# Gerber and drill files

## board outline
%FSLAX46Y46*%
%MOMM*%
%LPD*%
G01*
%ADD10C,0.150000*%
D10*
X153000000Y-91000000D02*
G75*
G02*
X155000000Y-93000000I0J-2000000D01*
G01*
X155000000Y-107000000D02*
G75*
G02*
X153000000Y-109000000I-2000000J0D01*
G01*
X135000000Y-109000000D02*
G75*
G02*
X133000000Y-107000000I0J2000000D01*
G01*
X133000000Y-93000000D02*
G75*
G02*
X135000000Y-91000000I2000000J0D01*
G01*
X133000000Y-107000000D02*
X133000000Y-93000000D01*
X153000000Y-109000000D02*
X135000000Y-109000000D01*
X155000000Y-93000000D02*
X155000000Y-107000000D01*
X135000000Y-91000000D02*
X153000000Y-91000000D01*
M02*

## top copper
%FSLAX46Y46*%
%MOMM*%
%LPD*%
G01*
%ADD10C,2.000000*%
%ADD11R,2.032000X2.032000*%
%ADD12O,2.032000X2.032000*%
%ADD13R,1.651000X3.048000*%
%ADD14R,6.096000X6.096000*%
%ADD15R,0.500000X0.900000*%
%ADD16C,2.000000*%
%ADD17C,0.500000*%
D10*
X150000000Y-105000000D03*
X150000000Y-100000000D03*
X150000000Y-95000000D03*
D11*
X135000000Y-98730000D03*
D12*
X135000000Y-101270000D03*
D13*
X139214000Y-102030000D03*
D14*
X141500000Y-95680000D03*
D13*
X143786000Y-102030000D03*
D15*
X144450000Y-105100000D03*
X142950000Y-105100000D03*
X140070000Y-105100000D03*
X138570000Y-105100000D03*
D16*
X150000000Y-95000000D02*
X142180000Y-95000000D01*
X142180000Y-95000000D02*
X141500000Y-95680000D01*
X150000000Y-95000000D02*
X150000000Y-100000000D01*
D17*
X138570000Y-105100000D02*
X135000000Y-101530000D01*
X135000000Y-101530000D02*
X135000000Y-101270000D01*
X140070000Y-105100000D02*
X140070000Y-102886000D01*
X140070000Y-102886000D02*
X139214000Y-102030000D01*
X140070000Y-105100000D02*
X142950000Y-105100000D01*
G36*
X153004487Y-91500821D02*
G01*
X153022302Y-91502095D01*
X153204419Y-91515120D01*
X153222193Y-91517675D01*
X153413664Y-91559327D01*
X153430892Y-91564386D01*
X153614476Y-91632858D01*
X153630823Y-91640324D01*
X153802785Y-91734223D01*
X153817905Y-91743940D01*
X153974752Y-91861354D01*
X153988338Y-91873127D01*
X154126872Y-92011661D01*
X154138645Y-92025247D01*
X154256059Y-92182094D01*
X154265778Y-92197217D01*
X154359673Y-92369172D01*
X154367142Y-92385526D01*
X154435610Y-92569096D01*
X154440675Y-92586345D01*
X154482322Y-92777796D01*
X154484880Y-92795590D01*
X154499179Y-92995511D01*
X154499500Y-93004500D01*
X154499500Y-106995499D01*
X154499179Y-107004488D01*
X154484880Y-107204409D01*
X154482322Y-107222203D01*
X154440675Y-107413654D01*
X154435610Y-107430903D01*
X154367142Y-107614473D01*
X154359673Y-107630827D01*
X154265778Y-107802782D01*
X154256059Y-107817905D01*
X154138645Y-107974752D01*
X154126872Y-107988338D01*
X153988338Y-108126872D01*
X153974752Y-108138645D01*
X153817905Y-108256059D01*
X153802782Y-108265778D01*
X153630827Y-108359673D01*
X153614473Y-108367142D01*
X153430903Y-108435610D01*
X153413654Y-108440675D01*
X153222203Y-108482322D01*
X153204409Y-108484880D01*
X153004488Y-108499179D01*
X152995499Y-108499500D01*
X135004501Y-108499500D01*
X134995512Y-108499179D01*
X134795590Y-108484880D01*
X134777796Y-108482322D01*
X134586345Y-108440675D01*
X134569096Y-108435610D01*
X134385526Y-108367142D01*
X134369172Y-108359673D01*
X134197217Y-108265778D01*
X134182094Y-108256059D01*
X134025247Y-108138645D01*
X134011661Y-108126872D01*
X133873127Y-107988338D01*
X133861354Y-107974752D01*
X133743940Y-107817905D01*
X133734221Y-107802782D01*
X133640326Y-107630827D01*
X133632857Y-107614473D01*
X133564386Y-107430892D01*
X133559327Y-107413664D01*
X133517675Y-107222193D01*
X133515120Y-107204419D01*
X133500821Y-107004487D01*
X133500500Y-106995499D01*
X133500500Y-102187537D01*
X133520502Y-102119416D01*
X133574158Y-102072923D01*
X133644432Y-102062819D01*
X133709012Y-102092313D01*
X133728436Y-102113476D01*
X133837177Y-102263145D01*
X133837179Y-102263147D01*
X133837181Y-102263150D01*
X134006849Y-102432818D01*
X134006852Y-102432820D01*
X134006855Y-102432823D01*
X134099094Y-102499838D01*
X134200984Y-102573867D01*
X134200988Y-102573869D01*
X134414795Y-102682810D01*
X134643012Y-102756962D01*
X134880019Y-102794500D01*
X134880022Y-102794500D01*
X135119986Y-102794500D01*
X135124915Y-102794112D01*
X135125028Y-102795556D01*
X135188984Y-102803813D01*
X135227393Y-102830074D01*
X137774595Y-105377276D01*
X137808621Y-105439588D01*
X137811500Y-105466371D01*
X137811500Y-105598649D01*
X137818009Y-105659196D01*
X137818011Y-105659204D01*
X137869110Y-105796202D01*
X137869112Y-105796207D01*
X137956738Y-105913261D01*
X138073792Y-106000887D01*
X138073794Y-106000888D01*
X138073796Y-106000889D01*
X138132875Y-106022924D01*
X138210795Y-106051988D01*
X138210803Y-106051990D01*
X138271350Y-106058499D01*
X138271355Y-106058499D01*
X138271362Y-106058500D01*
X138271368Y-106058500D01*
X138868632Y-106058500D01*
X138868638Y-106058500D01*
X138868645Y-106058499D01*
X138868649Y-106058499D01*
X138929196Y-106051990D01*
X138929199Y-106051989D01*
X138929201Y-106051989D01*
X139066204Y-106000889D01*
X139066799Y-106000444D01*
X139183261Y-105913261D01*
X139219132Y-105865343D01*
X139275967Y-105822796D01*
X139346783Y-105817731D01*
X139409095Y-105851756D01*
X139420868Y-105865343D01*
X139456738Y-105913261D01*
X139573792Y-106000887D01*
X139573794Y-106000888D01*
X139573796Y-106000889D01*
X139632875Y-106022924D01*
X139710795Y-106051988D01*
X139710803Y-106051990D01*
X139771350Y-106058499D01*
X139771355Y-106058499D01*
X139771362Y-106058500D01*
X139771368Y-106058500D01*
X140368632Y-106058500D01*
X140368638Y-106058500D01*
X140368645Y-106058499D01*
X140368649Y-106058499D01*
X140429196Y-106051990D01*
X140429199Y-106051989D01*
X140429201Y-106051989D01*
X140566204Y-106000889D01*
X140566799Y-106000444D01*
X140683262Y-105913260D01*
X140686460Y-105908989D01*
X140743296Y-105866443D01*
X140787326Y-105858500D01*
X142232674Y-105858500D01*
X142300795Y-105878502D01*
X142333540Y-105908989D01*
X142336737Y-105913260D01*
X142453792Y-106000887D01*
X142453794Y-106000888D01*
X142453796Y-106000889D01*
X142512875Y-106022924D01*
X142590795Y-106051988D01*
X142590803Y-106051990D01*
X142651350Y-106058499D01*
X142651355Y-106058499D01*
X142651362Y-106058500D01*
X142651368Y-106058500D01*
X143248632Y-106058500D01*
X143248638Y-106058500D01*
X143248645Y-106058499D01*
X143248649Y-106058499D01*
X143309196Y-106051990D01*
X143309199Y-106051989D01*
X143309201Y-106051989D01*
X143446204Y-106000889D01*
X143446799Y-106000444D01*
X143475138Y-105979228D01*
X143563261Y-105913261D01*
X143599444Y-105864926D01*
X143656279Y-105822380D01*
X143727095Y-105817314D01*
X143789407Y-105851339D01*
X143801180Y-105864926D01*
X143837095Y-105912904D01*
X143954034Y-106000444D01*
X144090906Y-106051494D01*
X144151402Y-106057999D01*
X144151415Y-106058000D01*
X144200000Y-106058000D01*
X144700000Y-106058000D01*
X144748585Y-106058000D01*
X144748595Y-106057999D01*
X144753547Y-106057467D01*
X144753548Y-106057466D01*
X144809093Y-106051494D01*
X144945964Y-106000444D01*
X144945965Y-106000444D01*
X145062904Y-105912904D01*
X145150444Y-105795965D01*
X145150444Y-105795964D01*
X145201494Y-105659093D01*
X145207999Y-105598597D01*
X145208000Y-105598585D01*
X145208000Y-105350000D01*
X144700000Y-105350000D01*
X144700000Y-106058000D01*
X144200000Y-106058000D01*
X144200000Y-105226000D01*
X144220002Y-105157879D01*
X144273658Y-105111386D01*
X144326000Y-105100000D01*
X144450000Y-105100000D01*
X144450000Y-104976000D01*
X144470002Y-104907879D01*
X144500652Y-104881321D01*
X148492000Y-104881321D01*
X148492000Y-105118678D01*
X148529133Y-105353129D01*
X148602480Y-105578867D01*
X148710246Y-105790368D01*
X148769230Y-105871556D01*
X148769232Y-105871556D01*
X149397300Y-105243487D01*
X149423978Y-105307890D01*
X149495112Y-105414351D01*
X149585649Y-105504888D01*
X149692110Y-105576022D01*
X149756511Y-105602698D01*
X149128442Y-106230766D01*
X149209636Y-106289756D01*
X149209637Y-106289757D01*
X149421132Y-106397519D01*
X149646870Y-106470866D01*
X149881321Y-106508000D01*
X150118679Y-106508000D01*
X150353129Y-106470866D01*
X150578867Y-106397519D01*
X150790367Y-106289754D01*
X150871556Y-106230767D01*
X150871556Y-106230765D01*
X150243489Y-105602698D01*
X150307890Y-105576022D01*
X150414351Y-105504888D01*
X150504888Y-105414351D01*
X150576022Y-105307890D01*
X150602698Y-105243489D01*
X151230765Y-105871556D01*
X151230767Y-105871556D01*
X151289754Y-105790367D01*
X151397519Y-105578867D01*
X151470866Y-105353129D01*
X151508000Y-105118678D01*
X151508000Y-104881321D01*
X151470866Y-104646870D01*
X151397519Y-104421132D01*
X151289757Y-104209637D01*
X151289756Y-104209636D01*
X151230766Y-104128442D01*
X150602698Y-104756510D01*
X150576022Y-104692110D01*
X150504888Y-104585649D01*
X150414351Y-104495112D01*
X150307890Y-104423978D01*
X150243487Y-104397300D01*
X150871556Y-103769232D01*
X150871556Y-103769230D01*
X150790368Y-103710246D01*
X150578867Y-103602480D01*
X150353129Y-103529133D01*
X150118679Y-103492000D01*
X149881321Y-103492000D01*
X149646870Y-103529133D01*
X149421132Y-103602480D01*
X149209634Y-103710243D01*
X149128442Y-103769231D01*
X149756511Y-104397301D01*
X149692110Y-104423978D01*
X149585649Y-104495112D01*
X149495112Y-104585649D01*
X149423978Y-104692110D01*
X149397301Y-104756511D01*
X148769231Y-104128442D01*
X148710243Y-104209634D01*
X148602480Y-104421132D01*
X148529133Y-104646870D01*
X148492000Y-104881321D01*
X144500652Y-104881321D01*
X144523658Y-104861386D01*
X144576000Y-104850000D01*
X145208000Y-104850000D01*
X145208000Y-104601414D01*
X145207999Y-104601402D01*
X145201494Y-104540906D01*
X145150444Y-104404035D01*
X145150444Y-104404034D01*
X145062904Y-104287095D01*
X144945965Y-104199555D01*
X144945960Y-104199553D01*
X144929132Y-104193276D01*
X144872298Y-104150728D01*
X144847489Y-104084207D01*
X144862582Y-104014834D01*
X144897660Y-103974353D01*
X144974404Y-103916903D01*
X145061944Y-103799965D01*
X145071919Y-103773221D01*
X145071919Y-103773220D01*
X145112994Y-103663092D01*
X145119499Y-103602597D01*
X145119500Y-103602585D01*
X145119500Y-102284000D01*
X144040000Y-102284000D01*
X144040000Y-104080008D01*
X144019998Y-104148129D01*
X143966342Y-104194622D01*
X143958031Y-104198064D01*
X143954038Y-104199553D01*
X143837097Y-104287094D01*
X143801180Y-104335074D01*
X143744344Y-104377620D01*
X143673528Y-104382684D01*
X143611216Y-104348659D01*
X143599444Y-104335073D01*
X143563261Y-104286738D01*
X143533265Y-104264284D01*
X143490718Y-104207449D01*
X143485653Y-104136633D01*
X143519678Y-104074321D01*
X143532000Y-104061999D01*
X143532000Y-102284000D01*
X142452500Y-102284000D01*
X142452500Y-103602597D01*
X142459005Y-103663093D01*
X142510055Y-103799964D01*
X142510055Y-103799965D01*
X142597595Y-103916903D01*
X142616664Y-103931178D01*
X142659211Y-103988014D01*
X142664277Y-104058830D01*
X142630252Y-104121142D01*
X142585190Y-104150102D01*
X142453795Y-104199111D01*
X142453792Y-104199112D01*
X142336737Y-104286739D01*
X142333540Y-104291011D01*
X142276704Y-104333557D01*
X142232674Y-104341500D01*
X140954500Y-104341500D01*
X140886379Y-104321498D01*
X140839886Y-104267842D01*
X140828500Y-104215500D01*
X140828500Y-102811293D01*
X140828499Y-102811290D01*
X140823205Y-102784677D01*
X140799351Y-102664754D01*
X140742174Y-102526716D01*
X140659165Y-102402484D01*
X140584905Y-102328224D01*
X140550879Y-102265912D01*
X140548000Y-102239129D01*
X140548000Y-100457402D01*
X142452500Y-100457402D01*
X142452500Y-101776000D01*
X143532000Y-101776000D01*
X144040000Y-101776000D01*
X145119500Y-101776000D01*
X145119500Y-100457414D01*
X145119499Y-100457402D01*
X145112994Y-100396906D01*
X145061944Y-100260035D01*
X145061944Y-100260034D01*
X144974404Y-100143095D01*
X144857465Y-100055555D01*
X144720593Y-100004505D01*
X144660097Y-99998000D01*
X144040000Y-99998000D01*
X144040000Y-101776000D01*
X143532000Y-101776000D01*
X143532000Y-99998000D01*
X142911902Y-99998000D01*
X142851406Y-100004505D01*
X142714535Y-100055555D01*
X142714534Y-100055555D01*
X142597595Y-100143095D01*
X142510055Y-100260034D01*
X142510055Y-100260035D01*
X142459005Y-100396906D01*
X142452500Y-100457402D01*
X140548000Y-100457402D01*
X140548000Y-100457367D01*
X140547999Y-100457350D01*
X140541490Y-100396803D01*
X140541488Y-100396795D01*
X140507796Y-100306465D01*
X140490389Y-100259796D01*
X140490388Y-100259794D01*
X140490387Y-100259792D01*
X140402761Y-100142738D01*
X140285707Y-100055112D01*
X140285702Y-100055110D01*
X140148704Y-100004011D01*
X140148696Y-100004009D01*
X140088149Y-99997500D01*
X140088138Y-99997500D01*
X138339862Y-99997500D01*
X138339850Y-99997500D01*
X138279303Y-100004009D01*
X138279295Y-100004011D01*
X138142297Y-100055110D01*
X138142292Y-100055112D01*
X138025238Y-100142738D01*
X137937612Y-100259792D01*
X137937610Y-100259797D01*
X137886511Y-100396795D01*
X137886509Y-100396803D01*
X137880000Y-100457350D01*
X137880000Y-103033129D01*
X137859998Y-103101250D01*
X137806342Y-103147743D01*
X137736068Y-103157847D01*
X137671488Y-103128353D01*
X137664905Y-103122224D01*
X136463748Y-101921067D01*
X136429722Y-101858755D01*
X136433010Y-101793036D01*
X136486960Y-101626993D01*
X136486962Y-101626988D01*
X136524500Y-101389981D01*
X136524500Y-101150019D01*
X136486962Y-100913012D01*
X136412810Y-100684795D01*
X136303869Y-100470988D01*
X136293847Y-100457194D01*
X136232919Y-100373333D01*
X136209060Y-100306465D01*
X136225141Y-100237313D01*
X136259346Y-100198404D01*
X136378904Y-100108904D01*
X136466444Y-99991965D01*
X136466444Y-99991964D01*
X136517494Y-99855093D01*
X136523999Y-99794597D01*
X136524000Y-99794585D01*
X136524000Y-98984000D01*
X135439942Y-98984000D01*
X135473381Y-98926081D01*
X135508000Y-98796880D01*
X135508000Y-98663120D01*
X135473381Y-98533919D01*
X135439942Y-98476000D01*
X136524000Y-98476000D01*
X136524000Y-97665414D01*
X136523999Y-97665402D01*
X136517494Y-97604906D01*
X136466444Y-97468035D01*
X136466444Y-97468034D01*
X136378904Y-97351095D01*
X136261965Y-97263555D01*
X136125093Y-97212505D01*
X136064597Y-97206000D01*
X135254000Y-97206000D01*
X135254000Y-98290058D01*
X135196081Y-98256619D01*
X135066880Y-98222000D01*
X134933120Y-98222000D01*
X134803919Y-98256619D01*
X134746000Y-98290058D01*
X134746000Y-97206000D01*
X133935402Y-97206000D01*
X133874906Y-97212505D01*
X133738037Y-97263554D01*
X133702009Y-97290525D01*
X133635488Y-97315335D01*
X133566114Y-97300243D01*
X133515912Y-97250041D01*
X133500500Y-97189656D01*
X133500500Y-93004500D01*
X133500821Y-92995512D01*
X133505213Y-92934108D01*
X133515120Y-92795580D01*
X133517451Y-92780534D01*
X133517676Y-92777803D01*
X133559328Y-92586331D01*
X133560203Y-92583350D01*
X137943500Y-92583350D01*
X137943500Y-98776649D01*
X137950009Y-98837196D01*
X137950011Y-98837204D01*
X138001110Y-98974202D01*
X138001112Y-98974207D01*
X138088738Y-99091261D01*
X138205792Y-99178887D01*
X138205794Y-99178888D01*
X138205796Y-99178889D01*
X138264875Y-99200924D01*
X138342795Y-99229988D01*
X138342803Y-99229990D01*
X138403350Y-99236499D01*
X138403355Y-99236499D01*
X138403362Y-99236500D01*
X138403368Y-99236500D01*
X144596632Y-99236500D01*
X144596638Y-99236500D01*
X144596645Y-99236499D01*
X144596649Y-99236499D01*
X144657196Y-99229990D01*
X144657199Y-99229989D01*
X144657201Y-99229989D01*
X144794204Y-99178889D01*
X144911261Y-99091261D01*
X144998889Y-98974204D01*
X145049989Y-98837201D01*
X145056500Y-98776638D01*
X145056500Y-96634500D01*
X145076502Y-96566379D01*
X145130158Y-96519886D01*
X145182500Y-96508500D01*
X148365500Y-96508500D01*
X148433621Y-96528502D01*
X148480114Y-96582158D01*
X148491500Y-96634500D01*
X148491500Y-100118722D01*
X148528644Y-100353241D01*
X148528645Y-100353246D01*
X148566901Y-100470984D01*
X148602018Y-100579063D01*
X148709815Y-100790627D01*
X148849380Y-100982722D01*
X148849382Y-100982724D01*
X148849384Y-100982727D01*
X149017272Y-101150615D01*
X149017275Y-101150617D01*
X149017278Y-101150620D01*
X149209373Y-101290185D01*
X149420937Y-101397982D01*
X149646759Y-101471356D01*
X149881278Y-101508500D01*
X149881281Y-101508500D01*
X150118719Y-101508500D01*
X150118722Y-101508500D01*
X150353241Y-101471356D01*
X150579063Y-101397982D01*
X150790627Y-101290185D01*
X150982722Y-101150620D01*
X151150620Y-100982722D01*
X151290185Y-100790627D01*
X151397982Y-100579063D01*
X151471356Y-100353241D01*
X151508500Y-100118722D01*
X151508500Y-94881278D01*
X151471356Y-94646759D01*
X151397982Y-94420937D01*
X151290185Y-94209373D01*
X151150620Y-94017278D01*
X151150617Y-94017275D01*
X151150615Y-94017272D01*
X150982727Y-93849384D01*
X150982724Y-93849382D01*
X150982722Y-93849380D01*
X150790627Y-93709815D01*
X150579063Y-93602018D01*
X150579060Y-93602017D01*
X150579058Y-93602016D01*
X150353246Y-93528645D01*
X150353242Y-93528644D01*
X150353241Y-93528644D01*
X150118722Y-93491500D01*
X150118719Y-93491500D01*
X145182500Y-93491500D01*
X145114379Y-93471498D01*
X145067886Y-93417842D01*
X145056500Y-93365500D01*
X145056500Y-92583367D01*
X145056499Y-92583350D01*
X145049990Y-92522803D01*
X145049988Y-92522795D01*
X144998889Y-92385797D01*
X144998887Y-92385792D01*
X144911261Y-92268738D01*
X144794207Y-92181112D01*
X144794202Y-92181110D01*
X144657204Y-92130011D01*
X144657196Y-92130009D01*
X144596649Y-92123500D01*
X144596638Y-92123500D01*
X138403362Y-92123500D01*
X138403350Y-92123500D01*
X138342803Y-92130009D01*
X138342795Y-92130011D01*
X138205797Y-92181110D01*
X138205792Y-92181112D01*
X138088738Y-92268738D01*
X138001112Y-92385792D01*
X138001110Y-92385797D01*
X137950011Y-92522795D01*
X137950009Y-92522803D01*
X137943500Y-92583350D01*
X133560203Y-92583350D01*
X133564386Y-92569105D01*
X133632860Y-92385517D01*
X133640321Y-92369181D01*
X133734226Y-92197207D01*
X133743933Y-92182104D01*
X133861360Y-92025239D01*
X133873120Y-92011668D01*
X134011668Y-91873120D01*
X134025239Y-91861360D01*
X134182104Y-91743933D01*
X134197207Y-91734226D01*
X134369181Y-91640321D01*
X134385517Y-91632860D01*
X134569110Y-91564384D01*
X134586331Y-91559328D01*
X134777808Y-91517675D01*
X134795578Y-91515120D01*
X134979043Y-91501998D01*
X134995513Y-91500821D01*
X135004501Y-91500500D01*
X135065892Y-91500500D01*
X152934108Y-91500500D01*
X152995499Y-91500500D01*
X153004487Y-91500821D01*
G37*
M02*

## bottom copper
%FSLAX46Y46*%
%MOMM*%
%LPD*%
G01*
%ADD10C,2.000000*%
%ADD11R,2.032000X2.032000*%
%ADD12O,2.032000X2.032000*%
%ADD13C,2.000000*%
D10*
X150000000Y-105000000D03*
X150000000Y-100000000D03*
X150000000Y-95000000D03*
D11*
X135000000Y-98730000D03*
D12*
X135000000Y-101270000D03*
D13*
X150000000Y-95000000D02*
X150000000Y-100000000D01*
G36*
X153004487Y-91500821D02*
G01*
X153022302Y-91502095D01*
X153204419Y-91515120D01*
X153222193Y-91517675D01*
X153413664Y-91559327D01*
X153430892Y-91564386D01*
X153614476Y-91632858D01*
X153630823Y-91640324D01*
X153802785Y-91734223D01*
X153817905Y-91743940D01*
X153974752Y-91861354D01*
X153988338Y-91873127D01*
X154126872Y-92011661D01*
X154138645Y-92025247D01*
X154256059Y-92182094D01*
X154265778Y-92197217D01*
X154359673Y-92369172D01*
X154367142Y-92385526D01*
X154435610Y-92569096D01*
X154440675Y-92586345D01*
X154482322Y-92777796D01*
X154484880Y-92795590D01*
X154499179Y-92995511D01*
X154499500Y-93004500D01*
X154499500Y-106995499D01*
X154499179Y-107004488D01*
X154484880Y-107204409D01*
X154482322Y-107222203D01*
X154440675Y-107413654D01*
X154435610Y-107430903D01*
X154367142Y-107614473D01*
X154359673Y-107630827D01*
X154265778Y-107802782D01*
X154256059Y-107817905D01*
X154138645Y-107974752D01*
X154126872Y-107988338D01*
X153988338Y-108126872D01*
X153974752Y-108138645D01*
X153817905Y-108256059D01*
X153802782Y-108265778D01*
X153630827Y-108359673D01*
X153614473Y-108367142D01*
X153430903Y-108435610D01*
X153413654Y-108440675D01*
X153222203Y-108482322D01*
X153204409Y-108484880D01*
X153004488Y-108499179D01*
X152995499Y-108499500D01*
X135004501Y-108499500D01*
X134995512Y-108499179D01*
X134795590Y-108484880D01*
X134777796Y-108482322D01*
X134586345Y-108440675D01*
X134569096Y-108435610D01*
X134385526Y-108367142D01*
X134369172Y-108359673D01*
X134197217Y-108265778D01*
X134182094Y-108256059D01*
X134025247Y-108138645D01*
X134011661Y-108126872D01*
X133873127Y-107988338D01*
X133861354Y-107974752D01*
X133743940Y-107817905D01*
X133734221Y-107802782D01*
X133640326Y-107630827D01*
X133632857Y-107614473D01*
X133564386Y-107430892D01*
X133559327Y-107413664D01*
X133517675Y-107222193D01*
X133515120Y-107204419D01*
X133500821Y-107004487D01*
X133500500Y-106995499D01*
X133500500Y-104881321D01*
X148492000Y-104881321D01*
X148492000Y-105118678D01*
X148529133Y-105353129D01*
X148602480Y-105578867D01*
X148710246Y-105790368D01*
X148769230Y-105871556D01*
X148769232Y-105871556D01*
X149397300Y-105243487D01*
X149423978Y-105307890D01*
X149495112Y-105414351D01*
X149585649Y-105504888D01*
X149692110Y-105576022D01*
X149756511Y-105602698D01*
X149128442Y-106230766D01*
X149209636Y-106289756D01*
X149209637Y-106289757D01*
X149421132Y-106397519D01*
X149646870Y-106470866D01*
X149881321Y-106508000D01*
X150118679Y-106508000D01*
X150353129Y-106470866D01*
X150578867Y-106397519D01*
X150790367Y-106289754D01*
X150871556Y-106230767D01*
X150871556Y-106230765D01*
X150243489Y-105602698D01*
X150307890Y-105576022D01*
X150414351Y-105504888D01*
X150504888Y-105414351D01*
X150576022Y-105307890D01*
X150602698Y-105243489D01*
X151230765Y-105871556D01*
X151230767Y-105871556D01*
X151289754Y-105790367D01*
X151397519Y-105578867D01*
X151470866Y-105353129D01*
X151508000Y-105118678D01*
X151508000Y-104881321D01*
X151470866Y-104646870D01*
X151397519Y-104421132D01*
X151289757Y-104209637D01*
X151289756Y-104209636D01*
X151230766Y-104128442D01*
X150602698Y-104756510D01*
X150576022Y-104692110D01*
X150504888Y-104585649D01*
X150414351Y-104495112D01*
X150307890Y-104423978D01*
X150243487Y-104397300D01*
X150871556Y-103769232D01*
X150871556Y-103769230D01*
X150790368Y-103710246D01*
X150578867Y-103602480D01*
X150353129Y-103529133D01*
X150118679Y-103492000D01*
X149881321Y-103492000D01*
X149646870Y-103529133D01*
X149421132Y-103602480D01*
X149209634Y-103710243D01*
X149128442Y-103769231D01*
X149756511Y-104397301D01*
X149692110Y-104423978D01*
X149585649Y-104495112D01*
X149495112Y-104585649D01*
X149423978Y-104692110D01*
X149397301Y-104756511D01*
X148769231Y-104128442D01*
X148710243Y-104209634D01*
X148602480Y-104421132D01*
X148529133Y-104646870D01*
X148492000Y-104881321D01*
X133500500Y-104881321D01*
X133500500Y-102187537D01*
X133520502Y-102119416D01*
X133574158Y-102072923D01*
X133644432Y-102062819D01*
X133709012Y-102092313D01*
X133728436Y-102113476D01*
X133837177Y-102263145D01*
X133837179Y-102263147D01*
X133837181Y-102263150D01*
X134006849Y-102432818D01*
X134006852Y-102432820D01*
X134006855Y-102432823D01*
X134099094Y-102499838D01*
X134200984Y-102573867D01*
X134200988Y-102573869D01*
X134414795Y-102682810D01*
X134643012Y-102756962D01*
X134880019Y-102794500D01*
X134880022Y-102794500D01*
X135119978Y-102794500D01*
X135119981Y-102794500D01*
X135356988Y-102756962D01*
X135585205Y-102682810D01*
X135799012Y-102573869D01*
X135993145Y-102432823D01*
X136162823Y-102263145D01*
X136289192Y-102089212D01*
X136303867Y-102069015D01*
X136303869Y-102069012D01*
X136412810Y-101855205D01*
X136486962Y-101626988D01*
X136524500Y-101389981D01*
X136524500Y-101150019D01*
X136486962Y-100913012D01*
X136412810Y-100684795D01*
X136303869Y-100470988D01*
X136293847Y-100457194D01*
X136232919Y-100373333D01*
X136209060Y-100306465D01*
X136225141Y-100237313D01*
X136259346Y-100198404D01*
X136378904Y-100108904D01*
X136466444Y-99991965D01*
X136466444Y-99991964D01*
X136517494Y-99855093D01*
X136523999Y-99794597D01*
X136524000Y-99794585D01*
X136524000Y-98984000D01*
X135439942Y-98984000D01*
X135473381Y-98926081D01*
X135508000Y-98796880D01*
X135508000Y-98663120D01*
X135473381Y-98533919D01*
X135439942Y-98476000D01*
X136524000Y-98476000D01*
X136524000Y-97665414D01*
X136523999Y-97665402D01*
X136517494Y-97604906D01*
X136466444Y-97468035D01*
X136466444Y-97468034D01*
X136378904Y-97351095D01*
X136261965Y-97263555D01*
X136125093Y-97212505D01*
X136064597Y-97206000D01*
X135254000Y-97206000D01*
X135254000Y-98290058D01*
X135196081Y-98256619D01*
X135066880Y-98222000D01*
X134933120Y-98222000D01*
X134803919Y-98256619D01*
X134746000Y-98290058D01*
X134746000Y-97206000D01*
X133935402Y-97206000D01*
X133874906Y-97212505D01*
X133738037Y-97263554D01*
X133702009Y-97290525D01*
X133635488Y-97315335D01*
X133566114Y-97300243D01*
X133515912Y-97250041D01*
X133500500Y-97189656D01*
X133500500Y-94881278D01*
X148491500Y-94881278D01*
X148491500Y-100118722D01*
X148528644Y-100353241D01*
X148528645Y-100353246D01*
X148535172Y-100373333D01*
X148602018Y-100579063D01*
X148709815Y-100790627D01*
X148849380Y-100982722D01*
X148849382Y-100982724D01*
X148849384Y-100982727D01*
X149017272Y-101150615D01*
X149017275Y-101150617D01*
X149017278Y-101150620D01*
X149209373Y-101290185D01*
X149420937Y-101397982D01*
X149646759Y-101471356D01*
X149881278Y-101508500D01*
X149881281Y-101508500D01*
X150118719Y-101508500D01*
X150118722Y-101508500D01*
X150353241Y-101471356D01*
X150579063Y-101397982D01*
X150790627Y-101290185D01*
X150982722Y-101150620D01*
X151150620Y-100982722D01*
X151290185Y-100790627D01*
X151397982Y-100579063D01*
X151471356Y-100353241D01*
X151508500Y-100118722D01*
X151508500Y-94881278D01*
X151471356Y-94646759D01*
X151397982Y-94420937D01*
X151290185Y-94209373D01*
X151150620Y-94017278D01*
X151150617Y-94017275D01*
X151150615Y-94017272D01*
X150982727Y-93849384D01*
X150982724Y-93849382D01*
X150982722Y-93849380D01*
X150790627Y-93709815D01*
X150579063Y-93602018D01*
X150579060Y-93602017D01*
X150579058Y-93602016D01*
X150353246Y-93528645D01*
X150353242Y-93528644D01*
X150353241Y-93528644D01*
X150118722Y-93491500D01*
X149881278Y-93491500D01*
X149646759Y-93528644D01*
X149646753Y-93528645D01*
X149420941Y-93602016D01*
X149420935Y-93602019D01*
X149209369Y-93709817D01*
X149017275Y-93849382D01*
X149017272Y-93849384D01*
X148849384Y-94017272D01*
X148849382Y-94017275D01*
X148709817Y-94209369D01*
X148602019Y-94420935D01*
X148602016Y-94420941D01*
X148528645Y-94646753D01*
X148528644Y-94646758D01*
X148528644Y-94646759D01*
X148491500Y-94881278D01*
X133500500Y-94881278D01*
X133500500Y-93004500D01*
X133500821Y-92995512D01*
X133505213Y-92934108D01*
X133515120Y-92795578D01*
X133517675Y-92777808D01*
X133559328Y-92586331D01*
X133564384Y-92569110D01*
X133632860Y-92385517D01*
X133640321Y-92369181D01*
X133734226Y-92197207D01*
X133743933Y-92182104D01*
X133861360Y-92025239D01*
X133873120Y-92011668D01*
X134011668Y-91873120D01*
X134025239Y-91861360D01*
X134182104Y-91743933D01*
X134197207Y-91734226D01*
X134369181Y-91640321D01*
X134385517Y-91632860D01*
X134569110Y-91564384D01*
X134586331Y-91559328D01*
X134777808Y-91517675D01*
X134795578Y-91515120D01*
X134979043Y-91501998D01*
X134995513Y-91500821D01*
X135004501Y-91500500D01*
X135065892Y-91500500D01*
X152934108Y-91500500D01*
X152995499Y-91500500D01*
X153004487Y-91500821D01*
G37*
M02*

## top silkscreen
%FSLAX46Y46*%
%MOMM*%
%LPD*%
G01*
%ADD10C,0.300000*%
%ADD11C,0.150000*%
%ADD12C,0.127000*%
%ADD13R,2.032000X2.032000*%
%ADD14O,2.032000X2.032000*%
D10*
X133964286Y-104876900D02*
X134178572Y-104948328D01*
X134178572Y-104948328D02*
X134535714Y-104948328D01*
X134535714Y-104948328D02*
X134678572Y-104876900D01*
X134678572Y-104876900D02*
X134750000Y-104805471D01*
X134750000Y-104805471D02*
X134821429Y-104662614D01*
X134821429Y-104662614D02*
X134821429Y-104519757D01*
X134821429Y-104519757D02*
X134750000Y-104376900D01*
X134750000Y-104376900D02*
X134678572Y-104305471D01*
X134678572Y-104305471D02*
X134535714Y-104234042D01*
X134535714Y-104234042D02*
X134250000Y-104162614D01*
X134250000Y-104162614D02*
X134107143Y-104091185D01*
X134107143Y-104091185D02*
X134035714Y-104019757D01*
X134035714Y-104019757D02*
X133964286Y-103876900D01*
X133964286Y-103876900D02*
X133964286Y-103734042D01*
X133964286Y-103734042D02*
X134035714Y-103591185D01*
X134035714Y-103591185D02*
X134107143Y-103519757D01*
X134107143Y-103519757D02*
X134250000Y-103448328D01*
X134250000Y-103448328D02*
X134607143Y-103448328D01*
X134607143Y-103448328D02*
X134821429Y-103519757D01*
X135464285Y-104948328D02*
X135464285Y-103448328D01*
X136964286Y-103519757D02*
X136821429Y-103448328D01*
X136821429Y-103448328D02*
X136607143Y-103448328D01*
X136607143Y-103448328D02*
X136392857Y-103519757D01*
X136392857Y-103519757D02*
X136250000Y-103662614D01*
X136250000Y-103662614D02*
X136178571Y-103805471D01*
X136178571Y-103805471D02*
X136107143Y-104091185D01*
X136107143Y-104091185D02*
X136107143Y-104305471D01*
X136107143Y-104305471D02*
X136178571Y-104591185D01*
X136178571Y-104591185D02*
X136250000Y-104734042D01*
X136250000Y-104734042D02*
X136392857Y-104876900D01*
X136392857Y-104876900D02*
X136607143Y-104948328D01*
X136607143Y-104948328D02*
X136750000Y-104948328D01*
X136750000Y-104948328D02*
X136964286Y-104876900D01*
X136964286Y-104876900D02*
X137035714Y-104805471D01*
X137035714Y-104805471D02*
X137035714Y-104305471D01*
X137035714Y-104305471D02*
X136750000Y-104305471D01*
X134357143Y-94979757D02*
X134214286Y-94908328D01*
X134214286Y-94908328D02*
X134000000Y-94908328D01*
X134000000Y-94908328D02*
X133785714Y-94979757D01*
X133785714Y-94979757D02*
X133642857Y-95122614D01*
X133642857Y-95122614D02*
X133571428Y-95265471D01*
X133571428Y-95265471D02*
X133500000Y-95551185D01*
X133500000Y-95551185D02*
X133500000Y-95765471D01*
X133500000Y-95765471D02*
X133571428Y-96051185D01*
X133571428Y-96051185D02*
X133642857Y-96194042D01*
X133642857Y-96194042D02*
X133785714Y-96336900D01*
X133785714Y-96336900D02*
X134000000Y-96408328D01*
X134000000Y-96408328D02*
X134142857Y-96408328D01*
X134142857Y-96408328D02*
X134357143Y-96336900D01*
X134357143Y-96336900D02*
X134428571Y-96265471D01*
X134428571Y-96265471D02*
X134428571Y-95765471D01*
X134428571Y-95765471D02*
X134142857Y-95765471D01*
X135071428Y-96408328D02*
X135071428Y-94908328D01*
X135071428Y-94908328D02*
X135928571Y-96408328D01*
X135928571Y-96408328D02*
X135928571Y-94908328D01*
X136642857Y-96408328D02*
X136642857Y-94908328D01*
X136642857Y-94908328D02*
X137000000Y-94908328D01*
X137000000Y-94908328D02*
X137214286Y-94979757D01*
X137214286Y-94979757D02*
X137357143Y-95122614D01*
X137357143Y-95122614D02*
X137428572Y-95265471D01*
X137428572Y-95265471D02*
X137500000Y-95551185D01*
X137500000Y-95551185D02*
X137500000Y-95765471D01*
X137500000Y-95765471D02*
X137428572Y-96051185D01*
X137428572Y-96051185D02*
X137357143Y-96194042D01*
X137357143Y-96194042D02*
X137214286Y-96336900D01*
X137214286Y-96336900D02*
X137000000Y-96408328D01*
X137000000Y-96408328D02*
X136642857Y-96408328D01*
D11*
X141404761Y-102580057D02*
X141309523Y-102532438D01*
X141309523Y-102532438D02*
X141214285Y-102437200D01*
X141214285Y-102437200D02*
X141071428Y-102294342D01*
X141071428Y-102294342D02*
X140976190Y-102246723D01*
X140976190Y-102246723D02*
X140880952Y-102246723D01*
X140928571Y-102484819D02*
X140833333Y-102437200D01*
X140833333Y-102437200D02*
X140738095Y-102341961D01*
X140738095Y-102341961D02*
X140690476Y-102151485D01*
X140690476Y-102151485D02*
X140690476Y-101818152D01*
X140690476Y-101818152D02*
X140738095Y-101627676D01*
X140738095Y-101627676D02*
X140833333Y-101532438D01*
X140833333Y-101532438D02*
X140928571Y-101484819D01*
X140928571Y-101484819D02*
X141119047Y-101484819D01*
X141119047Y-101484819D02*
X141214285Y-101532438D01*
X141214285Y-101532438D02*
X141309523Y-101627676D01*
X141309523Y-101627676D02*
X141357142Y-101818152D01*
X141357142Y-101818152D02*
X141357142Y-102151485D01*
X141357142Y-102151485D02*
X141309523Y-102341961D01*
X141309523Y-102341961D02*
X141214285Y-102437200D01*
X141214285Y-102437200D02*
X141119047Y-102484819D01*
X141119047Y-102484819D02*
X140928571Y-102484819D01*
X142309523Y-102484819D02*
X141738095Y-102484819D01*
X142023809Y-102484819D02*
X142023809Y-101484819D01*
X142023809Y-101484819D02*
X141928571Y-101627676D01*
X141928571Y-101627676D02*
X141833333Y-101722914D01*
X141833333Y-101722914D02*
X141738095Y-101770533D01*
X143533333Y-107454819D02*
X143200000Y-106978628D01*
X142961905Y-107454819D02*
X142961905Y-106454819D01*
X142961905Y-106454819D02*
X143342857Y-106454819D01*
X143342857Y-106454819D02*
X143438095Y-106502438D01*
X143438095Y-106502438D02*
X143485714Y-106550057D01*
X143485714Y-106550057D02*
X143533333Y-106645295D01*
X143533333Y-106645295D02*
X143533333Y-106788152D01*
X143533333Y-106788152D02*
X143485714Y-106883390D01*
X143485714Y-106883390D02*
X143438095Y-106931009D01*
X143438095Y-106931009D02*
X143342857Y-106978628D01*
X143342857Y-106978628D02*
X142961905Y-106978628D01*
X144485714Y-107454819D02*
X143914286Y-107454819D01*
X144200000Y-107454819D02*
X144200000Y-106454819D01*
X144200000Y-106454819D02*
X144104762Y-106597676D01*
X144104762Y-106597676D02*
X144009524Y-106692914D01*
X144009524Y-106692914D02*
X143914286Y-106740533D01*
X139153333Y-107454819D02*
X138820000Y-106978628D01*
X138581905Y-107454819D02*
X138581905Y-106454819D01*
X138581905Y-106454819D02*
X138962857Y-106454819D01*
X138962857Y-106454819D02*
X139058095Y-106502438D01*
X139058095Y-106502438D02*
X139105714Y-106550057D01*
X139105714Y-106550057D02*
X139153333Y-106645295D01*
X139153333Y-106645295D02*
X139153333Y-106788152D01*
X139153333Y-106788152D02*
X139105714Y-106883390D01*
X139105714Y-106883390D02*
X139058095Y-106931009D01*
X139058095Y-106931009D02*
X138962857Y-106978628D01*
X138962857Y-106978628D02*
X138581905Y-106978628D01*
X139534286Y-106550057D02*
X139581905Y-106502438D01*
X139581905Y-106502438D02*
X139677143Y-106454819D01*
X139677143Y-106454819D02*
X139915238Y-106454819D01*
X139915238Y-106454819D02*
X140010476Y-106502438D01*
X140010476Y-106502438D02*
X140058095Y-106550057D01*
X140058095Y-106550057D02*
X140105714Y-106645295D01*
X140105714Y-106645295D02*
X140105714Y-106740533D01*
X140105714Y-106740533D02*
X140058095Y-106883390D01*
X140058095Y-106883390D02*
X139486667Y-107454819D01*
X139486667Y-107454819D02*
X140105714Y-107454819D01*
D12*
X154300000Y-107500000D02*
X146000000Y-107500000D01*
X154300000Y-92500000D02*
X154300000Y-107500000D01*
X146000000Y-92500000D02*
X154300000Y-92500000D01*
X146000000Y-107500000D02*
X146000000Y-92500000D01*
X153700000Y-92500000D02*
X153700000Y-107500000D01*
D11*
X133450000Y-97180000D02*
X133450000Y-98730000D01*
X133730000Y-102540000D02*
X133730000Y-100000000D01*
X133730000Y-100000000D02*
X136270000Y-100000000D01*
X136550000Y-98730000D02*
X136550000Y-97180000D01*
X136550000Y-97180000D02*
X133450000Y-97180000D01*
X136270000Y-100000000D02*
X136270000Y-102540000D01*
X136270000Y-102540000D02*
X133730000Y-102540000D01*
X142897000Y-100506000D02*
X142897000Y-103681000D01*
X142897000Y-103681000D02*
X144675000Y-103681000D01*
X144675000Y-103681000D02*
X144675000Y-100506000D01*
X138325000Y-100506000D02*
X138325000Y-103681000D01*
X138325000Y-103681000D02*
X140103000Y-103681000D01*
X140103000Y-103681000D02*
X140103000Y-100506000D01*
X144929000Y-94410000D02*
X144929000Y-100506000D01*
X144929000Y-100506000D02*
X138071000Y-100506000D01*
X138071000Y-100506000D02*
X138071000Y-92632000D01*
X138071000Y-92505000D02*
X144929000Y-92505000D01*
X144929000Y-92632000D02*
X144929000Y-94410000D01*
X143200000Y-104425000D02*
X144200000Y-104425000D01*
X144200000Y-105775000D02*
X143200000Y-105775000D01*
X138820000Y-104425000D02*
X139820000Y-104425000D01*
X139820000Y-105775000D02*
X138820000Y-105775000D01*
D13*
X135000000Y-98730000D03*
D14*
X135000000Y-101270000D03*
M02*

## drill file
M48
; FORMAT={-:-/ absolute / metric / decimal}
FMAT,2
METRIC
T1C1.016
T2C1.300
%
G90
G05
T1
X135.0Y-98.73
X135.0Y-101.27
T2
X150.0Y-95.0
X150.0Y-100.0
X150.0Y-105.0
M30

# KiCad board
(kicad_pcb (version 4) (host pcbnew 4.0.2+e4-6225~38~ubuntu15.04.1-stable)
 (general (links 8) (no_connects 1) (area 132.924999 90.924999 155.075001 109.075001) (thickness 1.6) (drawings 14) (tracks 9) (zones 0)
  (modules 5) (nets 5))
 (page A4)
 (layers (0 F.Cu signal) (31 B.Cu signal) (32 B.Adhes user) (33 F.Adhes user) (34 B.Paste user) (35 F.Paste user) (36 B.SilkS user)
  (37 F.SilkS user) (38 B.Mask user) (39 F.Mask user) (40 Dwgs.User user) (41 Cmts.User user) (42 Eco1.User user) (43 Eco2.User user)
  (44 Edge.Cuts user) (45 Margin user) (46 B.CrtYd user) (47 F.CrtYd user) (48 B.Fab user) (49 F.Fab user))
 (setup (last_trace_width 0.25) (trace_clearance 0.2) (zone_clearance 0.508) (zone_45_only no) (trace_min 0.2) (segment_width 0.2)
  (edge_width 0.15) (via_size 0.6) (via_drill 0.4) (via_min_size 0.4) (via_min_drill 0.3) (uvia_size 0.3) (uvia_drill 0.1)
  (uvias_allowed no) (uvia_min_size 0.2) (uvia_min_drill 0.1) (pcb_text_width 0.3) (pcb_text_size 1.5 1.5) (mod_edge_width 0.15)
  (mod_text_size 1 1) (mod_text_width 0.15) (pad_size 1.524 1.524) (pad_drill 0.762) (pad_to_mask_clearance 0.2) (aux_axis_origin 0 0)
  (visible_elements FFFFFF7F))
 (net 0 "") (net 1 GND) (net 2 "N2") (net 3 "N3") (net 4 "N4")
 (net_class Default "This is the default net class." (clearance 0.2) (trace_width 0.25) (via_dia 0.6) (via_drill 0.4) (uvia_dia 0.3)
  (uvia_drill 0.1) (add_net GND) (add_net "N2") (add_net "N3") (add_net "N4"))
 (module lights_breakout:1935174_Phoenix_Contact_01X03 (layer F.Cu) (at 150 100 90)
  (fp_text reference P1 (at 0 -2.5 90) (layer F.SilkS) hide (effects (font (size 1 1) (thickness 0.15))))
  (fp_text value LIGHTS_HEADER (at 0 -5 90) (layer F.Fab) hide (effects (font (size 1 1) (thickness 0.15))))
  (fp_line (start -7.5 4.3) (end -7.5 -4) (layer F.SilkS) (width 0.127))
  (fp_line (start 7.5 4.3) (end -7.5 4.3) (layer F.SilkS) (width 0.127))
  (fp_line (start 7.5 -4) (end 7.5 4.3) (layer F.SilkS) (width 0.127))
  (fp_line (start -7.5 -4) (end 7.5 -4) (layer F.SilkS) (width 0.127))
  (fp_line (start 7.5 3.7) (end -7.5 3.7) (layer F.SilkS) (width 0.127))
  (pad 1 thru_hole circle (at -5 0 90) (size 2 2) (drill 1.3) (layers *.Cu *.Mask) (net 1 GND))
  (pad 2 thru_hole circle (at 0 0 90) (size 2 2) (drill 1.3) (layers *.Cu *.Mask) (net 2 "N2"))
  (pad 3 thru_hole circle (at 5 0 90) (size 2 2) (drill 1.3) (layers *.Cu *.Mask) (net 2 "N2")))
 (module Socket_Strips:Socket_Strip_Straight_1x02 (layer F.Cu) (at 135 98.73 270)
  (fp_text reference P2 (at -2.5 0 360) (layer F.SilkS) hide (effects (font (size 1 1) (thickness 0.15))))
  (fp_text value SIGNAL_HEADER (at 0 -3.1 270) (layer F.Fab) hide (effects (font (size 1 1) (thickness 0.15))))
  (fp_line (start -1.55 1.55) (end 0 1.55) (layer F.SilkS) (width 0.15))
  (fp_line (start 3.81 1.27) (end 1.27 1.27) (layer F.SilkS) (width 0.15))
  (fp_line (start 1.27 1.27) (end 1.27 -1.27) (layer F.SilkS) (width 0.15))
  (fp_line (start 0 -1.55) (end -1.55 -1.55) (layer F.SilkS) (width 0.15))
  (fp_line (start -1.55 -1.55) (end -1.55 1.55) (layer F.SilkS) (width 0.15))
  (fp_line (start 1.27 -1.27) (end 3.81 -1.27) (layer F.SilkS) (width 0.15))
  (fp_line (start 3.81 -1.27) (end 3.81 1.27) (layer F.SilkS) (width 0.15))
  (pad 1 thru_hole rect (at 0 0 270) (size 2.032 2.032) (drill 1.016) (layers *.Cu *.Mask F.SilkS) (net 1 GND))
  (pad 2 thru_hole oval (at 2.54 0 270) (size 2.032 2.032) (drill 1.016) (layers *.Cu *.Mask F.SilkS) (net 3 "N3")))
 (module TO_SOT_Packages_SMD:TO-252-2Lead (layer F.Cu) (at 141.5 102.03)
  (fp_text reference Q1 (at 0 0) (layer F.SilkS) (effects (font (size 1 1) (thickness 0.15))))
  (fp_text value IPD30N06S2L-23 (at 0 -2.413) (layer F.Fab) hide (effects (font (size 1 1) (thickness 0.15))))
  (fp_line (start 1.397 -1.524) (end 1.397 1.651) (layer F.SilkS) (width 0.15))
  (fp_line (start 1.397 1.651) (end 3.175 1.651) (layer F.SilkS) (width 0.15))
  (fp_line (start 3.175 1.651) (end 3.175 -1.524) (layer F.SilkS) (width 0.15))
  (fp_line (start -3.175 -1.524) (end -3.175 1.651) (layer F.SilkS) (width 0.15))
  (fp_line (start -3.175 1.651) (end -1.397 1.651) (layer F.SilkS) (width 0.15))
  (fp_line (start -1.397 1.651) (end -1.397 -1.524) (layer F.SilkS) (width 0.15))
  (fp_line (start 3.429 -7.62) (end 3.429 -1.524) (layer F.SilkS) (width 0.15))
  (fp_line (start 3.429 -1.524) (end -3.429 -1.524) (layer F.SilkS) (width 0.15))
  (fp_line (start -3.429 -1.524) (end -3.429 -9.398) (layer F.SilkS) (width 0.15))
  (fp_line (start -3.429 -9.525) (end 3.429 -9.525) (layer F.SilkS) (width 0.15))
  (fp_line (start 3.429 -9.398) (end 3.429 -7.62) (layer F.SilkS) (width 0.15))
  (pad 1 smd rect (at -2.286 0) (size 1.651 3.048) (layers F.Cu F.Paste F.Mask) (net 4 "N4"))
  (pad 2 smd rect (at 0 -6.35) (size 6.096 6.096) (layers F.Cu F.Paste F.Mask) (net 2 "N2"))
  (pad 3 smd rect (at 2.286 0) (size 1.651 3.048) (layers F.Cu F.Paste F.Mask) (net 1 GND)))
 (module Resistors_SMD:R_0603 (layer F.Cu) (at 143.7 105.1 180)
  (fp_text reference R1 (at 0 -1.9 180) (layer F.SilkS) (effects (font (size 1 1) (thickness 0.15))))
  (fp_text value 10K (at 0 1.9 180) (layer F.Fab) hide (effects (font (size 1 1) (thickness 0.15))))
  (fp_line (start 0.5 0.675) (end -0.5 0.675) (layer F.SilkS) (width 0.15))
  (fp_line (start -0.5 -0.675) (end 0.5 -0.675) (layer F.SilkS) (width 0.15))
  (pad 1 smd rect (at -0.75 0 180) (size 0.5 0.9) (layers F.Cu F.Paste F.Mask) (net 1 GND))
  (pad 2 smd rect (at 0.75 0 180) (size 0.5 0.9) (layers F.Cu F.Paste F.Mask) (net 4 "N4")))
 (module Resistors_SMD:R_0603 (layer F.Cu) (at 139.32 105.1 180)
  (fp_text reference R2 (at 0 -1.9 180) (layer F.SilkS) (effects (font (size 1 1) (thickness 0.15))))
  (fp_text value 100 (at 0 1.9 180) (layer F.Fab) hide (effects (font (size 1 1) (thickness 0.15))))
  (fp_line (start 0.5 0.675) (end -0.5 0.675) (layer F.SilkS) (width 0.15))
  (fp_line (start -0.5 -0.675) (end 0.5 -0.675) (layer F.SilkS) (width 0.15))
  (pad 1 smd rect (at -0.75 0 180) (size 0.5 0.9) (layers F.Cu F.Paste F.Mask) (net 4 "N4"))
  (pad 2 smd rect (at 0.75 0 180) (size 0.5 0.9) (layers F.Cu F.Paste F.Mask) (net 3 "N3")))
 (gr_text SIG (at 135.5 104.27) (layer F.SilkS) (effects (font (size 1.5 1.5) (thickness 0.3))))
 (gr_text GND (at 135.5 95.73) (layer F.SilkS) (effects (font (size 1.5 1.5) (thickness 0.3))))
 (gr_arc (start 153 93) (end 153 91) (angle 90) (layer Edge.Cuts) (width 0.15))
 (gr_arc (start 153 107) (end 155 107) (angle 90) (layer Edge.Cuts) (width 0.15))
 (gr_arc (start 135 107) (end 135 109) (angle 90) (layer Edge.Cuts) (width 0.15))
 (gr_arc (start 135 93) (end 133 93) (angle 90) (layer Edge.Cuts) (width 0.15))
 (gr_line (start 133 107) (end 133 93) (layer Edge.Cuts) (width 0.15))
 (gr_line (start 153 109) (end 135 109) (layer Edge.Cuts) (width 0.15))
 (gr_line (start 155 93) (end 155 107) (layer Edge.Cuts) (width 0.15))
 (gr_line (start 135 91) (end 153 91) (layer Edge.Cuts) (width 0.15))
 (segment (start 150 95) (end 142.18 95) (width 2) (layer F.Cu) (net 2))
 (segment (start 142.18 95) (end 141.5 95.68) (width 2) (layer F.Cu) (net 2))
 (segment (start 150 95) (end 150 100) (width 2) (layer B.Cu) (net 2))
 (segment (start 150 95) (end 150 100) (width 2) (layer F.Cu) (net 2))
 (segment (start 138.57 105.1) (end 135 101.53) (width 0.5) (layer F.Cu) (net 3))
 (segment (start 135 101.53) (end 135 101.27) (width 0.5) (layer F.Cu) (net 3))
 (segment (start 140.07 105.1) (end 140.07 102.886) (width 0.5) (layer F.Cu) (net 4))
 (segment (start 140.07 102.886) (end 139.214 102.03) (width 0.5) (layer F.Cu) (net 4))
 (segment (start 140.07 105.1) (end 142.95 105.1) (width 0.5) (layer F.Cu) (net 4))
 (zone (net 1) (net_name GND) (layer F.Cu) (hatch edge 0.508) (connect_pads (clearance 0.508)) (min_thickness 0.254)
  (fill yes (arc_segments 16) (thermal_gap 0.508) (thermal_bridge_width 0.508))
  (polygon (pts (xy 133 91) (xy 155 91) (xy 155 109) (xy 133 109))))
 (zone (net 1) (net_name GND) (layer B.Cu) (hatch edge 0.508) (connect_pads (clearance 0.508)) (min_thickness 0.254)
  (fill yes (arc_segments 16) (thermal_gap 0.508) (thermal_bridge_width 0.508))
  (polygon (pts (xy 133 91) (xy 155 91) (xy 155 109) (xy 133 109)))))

